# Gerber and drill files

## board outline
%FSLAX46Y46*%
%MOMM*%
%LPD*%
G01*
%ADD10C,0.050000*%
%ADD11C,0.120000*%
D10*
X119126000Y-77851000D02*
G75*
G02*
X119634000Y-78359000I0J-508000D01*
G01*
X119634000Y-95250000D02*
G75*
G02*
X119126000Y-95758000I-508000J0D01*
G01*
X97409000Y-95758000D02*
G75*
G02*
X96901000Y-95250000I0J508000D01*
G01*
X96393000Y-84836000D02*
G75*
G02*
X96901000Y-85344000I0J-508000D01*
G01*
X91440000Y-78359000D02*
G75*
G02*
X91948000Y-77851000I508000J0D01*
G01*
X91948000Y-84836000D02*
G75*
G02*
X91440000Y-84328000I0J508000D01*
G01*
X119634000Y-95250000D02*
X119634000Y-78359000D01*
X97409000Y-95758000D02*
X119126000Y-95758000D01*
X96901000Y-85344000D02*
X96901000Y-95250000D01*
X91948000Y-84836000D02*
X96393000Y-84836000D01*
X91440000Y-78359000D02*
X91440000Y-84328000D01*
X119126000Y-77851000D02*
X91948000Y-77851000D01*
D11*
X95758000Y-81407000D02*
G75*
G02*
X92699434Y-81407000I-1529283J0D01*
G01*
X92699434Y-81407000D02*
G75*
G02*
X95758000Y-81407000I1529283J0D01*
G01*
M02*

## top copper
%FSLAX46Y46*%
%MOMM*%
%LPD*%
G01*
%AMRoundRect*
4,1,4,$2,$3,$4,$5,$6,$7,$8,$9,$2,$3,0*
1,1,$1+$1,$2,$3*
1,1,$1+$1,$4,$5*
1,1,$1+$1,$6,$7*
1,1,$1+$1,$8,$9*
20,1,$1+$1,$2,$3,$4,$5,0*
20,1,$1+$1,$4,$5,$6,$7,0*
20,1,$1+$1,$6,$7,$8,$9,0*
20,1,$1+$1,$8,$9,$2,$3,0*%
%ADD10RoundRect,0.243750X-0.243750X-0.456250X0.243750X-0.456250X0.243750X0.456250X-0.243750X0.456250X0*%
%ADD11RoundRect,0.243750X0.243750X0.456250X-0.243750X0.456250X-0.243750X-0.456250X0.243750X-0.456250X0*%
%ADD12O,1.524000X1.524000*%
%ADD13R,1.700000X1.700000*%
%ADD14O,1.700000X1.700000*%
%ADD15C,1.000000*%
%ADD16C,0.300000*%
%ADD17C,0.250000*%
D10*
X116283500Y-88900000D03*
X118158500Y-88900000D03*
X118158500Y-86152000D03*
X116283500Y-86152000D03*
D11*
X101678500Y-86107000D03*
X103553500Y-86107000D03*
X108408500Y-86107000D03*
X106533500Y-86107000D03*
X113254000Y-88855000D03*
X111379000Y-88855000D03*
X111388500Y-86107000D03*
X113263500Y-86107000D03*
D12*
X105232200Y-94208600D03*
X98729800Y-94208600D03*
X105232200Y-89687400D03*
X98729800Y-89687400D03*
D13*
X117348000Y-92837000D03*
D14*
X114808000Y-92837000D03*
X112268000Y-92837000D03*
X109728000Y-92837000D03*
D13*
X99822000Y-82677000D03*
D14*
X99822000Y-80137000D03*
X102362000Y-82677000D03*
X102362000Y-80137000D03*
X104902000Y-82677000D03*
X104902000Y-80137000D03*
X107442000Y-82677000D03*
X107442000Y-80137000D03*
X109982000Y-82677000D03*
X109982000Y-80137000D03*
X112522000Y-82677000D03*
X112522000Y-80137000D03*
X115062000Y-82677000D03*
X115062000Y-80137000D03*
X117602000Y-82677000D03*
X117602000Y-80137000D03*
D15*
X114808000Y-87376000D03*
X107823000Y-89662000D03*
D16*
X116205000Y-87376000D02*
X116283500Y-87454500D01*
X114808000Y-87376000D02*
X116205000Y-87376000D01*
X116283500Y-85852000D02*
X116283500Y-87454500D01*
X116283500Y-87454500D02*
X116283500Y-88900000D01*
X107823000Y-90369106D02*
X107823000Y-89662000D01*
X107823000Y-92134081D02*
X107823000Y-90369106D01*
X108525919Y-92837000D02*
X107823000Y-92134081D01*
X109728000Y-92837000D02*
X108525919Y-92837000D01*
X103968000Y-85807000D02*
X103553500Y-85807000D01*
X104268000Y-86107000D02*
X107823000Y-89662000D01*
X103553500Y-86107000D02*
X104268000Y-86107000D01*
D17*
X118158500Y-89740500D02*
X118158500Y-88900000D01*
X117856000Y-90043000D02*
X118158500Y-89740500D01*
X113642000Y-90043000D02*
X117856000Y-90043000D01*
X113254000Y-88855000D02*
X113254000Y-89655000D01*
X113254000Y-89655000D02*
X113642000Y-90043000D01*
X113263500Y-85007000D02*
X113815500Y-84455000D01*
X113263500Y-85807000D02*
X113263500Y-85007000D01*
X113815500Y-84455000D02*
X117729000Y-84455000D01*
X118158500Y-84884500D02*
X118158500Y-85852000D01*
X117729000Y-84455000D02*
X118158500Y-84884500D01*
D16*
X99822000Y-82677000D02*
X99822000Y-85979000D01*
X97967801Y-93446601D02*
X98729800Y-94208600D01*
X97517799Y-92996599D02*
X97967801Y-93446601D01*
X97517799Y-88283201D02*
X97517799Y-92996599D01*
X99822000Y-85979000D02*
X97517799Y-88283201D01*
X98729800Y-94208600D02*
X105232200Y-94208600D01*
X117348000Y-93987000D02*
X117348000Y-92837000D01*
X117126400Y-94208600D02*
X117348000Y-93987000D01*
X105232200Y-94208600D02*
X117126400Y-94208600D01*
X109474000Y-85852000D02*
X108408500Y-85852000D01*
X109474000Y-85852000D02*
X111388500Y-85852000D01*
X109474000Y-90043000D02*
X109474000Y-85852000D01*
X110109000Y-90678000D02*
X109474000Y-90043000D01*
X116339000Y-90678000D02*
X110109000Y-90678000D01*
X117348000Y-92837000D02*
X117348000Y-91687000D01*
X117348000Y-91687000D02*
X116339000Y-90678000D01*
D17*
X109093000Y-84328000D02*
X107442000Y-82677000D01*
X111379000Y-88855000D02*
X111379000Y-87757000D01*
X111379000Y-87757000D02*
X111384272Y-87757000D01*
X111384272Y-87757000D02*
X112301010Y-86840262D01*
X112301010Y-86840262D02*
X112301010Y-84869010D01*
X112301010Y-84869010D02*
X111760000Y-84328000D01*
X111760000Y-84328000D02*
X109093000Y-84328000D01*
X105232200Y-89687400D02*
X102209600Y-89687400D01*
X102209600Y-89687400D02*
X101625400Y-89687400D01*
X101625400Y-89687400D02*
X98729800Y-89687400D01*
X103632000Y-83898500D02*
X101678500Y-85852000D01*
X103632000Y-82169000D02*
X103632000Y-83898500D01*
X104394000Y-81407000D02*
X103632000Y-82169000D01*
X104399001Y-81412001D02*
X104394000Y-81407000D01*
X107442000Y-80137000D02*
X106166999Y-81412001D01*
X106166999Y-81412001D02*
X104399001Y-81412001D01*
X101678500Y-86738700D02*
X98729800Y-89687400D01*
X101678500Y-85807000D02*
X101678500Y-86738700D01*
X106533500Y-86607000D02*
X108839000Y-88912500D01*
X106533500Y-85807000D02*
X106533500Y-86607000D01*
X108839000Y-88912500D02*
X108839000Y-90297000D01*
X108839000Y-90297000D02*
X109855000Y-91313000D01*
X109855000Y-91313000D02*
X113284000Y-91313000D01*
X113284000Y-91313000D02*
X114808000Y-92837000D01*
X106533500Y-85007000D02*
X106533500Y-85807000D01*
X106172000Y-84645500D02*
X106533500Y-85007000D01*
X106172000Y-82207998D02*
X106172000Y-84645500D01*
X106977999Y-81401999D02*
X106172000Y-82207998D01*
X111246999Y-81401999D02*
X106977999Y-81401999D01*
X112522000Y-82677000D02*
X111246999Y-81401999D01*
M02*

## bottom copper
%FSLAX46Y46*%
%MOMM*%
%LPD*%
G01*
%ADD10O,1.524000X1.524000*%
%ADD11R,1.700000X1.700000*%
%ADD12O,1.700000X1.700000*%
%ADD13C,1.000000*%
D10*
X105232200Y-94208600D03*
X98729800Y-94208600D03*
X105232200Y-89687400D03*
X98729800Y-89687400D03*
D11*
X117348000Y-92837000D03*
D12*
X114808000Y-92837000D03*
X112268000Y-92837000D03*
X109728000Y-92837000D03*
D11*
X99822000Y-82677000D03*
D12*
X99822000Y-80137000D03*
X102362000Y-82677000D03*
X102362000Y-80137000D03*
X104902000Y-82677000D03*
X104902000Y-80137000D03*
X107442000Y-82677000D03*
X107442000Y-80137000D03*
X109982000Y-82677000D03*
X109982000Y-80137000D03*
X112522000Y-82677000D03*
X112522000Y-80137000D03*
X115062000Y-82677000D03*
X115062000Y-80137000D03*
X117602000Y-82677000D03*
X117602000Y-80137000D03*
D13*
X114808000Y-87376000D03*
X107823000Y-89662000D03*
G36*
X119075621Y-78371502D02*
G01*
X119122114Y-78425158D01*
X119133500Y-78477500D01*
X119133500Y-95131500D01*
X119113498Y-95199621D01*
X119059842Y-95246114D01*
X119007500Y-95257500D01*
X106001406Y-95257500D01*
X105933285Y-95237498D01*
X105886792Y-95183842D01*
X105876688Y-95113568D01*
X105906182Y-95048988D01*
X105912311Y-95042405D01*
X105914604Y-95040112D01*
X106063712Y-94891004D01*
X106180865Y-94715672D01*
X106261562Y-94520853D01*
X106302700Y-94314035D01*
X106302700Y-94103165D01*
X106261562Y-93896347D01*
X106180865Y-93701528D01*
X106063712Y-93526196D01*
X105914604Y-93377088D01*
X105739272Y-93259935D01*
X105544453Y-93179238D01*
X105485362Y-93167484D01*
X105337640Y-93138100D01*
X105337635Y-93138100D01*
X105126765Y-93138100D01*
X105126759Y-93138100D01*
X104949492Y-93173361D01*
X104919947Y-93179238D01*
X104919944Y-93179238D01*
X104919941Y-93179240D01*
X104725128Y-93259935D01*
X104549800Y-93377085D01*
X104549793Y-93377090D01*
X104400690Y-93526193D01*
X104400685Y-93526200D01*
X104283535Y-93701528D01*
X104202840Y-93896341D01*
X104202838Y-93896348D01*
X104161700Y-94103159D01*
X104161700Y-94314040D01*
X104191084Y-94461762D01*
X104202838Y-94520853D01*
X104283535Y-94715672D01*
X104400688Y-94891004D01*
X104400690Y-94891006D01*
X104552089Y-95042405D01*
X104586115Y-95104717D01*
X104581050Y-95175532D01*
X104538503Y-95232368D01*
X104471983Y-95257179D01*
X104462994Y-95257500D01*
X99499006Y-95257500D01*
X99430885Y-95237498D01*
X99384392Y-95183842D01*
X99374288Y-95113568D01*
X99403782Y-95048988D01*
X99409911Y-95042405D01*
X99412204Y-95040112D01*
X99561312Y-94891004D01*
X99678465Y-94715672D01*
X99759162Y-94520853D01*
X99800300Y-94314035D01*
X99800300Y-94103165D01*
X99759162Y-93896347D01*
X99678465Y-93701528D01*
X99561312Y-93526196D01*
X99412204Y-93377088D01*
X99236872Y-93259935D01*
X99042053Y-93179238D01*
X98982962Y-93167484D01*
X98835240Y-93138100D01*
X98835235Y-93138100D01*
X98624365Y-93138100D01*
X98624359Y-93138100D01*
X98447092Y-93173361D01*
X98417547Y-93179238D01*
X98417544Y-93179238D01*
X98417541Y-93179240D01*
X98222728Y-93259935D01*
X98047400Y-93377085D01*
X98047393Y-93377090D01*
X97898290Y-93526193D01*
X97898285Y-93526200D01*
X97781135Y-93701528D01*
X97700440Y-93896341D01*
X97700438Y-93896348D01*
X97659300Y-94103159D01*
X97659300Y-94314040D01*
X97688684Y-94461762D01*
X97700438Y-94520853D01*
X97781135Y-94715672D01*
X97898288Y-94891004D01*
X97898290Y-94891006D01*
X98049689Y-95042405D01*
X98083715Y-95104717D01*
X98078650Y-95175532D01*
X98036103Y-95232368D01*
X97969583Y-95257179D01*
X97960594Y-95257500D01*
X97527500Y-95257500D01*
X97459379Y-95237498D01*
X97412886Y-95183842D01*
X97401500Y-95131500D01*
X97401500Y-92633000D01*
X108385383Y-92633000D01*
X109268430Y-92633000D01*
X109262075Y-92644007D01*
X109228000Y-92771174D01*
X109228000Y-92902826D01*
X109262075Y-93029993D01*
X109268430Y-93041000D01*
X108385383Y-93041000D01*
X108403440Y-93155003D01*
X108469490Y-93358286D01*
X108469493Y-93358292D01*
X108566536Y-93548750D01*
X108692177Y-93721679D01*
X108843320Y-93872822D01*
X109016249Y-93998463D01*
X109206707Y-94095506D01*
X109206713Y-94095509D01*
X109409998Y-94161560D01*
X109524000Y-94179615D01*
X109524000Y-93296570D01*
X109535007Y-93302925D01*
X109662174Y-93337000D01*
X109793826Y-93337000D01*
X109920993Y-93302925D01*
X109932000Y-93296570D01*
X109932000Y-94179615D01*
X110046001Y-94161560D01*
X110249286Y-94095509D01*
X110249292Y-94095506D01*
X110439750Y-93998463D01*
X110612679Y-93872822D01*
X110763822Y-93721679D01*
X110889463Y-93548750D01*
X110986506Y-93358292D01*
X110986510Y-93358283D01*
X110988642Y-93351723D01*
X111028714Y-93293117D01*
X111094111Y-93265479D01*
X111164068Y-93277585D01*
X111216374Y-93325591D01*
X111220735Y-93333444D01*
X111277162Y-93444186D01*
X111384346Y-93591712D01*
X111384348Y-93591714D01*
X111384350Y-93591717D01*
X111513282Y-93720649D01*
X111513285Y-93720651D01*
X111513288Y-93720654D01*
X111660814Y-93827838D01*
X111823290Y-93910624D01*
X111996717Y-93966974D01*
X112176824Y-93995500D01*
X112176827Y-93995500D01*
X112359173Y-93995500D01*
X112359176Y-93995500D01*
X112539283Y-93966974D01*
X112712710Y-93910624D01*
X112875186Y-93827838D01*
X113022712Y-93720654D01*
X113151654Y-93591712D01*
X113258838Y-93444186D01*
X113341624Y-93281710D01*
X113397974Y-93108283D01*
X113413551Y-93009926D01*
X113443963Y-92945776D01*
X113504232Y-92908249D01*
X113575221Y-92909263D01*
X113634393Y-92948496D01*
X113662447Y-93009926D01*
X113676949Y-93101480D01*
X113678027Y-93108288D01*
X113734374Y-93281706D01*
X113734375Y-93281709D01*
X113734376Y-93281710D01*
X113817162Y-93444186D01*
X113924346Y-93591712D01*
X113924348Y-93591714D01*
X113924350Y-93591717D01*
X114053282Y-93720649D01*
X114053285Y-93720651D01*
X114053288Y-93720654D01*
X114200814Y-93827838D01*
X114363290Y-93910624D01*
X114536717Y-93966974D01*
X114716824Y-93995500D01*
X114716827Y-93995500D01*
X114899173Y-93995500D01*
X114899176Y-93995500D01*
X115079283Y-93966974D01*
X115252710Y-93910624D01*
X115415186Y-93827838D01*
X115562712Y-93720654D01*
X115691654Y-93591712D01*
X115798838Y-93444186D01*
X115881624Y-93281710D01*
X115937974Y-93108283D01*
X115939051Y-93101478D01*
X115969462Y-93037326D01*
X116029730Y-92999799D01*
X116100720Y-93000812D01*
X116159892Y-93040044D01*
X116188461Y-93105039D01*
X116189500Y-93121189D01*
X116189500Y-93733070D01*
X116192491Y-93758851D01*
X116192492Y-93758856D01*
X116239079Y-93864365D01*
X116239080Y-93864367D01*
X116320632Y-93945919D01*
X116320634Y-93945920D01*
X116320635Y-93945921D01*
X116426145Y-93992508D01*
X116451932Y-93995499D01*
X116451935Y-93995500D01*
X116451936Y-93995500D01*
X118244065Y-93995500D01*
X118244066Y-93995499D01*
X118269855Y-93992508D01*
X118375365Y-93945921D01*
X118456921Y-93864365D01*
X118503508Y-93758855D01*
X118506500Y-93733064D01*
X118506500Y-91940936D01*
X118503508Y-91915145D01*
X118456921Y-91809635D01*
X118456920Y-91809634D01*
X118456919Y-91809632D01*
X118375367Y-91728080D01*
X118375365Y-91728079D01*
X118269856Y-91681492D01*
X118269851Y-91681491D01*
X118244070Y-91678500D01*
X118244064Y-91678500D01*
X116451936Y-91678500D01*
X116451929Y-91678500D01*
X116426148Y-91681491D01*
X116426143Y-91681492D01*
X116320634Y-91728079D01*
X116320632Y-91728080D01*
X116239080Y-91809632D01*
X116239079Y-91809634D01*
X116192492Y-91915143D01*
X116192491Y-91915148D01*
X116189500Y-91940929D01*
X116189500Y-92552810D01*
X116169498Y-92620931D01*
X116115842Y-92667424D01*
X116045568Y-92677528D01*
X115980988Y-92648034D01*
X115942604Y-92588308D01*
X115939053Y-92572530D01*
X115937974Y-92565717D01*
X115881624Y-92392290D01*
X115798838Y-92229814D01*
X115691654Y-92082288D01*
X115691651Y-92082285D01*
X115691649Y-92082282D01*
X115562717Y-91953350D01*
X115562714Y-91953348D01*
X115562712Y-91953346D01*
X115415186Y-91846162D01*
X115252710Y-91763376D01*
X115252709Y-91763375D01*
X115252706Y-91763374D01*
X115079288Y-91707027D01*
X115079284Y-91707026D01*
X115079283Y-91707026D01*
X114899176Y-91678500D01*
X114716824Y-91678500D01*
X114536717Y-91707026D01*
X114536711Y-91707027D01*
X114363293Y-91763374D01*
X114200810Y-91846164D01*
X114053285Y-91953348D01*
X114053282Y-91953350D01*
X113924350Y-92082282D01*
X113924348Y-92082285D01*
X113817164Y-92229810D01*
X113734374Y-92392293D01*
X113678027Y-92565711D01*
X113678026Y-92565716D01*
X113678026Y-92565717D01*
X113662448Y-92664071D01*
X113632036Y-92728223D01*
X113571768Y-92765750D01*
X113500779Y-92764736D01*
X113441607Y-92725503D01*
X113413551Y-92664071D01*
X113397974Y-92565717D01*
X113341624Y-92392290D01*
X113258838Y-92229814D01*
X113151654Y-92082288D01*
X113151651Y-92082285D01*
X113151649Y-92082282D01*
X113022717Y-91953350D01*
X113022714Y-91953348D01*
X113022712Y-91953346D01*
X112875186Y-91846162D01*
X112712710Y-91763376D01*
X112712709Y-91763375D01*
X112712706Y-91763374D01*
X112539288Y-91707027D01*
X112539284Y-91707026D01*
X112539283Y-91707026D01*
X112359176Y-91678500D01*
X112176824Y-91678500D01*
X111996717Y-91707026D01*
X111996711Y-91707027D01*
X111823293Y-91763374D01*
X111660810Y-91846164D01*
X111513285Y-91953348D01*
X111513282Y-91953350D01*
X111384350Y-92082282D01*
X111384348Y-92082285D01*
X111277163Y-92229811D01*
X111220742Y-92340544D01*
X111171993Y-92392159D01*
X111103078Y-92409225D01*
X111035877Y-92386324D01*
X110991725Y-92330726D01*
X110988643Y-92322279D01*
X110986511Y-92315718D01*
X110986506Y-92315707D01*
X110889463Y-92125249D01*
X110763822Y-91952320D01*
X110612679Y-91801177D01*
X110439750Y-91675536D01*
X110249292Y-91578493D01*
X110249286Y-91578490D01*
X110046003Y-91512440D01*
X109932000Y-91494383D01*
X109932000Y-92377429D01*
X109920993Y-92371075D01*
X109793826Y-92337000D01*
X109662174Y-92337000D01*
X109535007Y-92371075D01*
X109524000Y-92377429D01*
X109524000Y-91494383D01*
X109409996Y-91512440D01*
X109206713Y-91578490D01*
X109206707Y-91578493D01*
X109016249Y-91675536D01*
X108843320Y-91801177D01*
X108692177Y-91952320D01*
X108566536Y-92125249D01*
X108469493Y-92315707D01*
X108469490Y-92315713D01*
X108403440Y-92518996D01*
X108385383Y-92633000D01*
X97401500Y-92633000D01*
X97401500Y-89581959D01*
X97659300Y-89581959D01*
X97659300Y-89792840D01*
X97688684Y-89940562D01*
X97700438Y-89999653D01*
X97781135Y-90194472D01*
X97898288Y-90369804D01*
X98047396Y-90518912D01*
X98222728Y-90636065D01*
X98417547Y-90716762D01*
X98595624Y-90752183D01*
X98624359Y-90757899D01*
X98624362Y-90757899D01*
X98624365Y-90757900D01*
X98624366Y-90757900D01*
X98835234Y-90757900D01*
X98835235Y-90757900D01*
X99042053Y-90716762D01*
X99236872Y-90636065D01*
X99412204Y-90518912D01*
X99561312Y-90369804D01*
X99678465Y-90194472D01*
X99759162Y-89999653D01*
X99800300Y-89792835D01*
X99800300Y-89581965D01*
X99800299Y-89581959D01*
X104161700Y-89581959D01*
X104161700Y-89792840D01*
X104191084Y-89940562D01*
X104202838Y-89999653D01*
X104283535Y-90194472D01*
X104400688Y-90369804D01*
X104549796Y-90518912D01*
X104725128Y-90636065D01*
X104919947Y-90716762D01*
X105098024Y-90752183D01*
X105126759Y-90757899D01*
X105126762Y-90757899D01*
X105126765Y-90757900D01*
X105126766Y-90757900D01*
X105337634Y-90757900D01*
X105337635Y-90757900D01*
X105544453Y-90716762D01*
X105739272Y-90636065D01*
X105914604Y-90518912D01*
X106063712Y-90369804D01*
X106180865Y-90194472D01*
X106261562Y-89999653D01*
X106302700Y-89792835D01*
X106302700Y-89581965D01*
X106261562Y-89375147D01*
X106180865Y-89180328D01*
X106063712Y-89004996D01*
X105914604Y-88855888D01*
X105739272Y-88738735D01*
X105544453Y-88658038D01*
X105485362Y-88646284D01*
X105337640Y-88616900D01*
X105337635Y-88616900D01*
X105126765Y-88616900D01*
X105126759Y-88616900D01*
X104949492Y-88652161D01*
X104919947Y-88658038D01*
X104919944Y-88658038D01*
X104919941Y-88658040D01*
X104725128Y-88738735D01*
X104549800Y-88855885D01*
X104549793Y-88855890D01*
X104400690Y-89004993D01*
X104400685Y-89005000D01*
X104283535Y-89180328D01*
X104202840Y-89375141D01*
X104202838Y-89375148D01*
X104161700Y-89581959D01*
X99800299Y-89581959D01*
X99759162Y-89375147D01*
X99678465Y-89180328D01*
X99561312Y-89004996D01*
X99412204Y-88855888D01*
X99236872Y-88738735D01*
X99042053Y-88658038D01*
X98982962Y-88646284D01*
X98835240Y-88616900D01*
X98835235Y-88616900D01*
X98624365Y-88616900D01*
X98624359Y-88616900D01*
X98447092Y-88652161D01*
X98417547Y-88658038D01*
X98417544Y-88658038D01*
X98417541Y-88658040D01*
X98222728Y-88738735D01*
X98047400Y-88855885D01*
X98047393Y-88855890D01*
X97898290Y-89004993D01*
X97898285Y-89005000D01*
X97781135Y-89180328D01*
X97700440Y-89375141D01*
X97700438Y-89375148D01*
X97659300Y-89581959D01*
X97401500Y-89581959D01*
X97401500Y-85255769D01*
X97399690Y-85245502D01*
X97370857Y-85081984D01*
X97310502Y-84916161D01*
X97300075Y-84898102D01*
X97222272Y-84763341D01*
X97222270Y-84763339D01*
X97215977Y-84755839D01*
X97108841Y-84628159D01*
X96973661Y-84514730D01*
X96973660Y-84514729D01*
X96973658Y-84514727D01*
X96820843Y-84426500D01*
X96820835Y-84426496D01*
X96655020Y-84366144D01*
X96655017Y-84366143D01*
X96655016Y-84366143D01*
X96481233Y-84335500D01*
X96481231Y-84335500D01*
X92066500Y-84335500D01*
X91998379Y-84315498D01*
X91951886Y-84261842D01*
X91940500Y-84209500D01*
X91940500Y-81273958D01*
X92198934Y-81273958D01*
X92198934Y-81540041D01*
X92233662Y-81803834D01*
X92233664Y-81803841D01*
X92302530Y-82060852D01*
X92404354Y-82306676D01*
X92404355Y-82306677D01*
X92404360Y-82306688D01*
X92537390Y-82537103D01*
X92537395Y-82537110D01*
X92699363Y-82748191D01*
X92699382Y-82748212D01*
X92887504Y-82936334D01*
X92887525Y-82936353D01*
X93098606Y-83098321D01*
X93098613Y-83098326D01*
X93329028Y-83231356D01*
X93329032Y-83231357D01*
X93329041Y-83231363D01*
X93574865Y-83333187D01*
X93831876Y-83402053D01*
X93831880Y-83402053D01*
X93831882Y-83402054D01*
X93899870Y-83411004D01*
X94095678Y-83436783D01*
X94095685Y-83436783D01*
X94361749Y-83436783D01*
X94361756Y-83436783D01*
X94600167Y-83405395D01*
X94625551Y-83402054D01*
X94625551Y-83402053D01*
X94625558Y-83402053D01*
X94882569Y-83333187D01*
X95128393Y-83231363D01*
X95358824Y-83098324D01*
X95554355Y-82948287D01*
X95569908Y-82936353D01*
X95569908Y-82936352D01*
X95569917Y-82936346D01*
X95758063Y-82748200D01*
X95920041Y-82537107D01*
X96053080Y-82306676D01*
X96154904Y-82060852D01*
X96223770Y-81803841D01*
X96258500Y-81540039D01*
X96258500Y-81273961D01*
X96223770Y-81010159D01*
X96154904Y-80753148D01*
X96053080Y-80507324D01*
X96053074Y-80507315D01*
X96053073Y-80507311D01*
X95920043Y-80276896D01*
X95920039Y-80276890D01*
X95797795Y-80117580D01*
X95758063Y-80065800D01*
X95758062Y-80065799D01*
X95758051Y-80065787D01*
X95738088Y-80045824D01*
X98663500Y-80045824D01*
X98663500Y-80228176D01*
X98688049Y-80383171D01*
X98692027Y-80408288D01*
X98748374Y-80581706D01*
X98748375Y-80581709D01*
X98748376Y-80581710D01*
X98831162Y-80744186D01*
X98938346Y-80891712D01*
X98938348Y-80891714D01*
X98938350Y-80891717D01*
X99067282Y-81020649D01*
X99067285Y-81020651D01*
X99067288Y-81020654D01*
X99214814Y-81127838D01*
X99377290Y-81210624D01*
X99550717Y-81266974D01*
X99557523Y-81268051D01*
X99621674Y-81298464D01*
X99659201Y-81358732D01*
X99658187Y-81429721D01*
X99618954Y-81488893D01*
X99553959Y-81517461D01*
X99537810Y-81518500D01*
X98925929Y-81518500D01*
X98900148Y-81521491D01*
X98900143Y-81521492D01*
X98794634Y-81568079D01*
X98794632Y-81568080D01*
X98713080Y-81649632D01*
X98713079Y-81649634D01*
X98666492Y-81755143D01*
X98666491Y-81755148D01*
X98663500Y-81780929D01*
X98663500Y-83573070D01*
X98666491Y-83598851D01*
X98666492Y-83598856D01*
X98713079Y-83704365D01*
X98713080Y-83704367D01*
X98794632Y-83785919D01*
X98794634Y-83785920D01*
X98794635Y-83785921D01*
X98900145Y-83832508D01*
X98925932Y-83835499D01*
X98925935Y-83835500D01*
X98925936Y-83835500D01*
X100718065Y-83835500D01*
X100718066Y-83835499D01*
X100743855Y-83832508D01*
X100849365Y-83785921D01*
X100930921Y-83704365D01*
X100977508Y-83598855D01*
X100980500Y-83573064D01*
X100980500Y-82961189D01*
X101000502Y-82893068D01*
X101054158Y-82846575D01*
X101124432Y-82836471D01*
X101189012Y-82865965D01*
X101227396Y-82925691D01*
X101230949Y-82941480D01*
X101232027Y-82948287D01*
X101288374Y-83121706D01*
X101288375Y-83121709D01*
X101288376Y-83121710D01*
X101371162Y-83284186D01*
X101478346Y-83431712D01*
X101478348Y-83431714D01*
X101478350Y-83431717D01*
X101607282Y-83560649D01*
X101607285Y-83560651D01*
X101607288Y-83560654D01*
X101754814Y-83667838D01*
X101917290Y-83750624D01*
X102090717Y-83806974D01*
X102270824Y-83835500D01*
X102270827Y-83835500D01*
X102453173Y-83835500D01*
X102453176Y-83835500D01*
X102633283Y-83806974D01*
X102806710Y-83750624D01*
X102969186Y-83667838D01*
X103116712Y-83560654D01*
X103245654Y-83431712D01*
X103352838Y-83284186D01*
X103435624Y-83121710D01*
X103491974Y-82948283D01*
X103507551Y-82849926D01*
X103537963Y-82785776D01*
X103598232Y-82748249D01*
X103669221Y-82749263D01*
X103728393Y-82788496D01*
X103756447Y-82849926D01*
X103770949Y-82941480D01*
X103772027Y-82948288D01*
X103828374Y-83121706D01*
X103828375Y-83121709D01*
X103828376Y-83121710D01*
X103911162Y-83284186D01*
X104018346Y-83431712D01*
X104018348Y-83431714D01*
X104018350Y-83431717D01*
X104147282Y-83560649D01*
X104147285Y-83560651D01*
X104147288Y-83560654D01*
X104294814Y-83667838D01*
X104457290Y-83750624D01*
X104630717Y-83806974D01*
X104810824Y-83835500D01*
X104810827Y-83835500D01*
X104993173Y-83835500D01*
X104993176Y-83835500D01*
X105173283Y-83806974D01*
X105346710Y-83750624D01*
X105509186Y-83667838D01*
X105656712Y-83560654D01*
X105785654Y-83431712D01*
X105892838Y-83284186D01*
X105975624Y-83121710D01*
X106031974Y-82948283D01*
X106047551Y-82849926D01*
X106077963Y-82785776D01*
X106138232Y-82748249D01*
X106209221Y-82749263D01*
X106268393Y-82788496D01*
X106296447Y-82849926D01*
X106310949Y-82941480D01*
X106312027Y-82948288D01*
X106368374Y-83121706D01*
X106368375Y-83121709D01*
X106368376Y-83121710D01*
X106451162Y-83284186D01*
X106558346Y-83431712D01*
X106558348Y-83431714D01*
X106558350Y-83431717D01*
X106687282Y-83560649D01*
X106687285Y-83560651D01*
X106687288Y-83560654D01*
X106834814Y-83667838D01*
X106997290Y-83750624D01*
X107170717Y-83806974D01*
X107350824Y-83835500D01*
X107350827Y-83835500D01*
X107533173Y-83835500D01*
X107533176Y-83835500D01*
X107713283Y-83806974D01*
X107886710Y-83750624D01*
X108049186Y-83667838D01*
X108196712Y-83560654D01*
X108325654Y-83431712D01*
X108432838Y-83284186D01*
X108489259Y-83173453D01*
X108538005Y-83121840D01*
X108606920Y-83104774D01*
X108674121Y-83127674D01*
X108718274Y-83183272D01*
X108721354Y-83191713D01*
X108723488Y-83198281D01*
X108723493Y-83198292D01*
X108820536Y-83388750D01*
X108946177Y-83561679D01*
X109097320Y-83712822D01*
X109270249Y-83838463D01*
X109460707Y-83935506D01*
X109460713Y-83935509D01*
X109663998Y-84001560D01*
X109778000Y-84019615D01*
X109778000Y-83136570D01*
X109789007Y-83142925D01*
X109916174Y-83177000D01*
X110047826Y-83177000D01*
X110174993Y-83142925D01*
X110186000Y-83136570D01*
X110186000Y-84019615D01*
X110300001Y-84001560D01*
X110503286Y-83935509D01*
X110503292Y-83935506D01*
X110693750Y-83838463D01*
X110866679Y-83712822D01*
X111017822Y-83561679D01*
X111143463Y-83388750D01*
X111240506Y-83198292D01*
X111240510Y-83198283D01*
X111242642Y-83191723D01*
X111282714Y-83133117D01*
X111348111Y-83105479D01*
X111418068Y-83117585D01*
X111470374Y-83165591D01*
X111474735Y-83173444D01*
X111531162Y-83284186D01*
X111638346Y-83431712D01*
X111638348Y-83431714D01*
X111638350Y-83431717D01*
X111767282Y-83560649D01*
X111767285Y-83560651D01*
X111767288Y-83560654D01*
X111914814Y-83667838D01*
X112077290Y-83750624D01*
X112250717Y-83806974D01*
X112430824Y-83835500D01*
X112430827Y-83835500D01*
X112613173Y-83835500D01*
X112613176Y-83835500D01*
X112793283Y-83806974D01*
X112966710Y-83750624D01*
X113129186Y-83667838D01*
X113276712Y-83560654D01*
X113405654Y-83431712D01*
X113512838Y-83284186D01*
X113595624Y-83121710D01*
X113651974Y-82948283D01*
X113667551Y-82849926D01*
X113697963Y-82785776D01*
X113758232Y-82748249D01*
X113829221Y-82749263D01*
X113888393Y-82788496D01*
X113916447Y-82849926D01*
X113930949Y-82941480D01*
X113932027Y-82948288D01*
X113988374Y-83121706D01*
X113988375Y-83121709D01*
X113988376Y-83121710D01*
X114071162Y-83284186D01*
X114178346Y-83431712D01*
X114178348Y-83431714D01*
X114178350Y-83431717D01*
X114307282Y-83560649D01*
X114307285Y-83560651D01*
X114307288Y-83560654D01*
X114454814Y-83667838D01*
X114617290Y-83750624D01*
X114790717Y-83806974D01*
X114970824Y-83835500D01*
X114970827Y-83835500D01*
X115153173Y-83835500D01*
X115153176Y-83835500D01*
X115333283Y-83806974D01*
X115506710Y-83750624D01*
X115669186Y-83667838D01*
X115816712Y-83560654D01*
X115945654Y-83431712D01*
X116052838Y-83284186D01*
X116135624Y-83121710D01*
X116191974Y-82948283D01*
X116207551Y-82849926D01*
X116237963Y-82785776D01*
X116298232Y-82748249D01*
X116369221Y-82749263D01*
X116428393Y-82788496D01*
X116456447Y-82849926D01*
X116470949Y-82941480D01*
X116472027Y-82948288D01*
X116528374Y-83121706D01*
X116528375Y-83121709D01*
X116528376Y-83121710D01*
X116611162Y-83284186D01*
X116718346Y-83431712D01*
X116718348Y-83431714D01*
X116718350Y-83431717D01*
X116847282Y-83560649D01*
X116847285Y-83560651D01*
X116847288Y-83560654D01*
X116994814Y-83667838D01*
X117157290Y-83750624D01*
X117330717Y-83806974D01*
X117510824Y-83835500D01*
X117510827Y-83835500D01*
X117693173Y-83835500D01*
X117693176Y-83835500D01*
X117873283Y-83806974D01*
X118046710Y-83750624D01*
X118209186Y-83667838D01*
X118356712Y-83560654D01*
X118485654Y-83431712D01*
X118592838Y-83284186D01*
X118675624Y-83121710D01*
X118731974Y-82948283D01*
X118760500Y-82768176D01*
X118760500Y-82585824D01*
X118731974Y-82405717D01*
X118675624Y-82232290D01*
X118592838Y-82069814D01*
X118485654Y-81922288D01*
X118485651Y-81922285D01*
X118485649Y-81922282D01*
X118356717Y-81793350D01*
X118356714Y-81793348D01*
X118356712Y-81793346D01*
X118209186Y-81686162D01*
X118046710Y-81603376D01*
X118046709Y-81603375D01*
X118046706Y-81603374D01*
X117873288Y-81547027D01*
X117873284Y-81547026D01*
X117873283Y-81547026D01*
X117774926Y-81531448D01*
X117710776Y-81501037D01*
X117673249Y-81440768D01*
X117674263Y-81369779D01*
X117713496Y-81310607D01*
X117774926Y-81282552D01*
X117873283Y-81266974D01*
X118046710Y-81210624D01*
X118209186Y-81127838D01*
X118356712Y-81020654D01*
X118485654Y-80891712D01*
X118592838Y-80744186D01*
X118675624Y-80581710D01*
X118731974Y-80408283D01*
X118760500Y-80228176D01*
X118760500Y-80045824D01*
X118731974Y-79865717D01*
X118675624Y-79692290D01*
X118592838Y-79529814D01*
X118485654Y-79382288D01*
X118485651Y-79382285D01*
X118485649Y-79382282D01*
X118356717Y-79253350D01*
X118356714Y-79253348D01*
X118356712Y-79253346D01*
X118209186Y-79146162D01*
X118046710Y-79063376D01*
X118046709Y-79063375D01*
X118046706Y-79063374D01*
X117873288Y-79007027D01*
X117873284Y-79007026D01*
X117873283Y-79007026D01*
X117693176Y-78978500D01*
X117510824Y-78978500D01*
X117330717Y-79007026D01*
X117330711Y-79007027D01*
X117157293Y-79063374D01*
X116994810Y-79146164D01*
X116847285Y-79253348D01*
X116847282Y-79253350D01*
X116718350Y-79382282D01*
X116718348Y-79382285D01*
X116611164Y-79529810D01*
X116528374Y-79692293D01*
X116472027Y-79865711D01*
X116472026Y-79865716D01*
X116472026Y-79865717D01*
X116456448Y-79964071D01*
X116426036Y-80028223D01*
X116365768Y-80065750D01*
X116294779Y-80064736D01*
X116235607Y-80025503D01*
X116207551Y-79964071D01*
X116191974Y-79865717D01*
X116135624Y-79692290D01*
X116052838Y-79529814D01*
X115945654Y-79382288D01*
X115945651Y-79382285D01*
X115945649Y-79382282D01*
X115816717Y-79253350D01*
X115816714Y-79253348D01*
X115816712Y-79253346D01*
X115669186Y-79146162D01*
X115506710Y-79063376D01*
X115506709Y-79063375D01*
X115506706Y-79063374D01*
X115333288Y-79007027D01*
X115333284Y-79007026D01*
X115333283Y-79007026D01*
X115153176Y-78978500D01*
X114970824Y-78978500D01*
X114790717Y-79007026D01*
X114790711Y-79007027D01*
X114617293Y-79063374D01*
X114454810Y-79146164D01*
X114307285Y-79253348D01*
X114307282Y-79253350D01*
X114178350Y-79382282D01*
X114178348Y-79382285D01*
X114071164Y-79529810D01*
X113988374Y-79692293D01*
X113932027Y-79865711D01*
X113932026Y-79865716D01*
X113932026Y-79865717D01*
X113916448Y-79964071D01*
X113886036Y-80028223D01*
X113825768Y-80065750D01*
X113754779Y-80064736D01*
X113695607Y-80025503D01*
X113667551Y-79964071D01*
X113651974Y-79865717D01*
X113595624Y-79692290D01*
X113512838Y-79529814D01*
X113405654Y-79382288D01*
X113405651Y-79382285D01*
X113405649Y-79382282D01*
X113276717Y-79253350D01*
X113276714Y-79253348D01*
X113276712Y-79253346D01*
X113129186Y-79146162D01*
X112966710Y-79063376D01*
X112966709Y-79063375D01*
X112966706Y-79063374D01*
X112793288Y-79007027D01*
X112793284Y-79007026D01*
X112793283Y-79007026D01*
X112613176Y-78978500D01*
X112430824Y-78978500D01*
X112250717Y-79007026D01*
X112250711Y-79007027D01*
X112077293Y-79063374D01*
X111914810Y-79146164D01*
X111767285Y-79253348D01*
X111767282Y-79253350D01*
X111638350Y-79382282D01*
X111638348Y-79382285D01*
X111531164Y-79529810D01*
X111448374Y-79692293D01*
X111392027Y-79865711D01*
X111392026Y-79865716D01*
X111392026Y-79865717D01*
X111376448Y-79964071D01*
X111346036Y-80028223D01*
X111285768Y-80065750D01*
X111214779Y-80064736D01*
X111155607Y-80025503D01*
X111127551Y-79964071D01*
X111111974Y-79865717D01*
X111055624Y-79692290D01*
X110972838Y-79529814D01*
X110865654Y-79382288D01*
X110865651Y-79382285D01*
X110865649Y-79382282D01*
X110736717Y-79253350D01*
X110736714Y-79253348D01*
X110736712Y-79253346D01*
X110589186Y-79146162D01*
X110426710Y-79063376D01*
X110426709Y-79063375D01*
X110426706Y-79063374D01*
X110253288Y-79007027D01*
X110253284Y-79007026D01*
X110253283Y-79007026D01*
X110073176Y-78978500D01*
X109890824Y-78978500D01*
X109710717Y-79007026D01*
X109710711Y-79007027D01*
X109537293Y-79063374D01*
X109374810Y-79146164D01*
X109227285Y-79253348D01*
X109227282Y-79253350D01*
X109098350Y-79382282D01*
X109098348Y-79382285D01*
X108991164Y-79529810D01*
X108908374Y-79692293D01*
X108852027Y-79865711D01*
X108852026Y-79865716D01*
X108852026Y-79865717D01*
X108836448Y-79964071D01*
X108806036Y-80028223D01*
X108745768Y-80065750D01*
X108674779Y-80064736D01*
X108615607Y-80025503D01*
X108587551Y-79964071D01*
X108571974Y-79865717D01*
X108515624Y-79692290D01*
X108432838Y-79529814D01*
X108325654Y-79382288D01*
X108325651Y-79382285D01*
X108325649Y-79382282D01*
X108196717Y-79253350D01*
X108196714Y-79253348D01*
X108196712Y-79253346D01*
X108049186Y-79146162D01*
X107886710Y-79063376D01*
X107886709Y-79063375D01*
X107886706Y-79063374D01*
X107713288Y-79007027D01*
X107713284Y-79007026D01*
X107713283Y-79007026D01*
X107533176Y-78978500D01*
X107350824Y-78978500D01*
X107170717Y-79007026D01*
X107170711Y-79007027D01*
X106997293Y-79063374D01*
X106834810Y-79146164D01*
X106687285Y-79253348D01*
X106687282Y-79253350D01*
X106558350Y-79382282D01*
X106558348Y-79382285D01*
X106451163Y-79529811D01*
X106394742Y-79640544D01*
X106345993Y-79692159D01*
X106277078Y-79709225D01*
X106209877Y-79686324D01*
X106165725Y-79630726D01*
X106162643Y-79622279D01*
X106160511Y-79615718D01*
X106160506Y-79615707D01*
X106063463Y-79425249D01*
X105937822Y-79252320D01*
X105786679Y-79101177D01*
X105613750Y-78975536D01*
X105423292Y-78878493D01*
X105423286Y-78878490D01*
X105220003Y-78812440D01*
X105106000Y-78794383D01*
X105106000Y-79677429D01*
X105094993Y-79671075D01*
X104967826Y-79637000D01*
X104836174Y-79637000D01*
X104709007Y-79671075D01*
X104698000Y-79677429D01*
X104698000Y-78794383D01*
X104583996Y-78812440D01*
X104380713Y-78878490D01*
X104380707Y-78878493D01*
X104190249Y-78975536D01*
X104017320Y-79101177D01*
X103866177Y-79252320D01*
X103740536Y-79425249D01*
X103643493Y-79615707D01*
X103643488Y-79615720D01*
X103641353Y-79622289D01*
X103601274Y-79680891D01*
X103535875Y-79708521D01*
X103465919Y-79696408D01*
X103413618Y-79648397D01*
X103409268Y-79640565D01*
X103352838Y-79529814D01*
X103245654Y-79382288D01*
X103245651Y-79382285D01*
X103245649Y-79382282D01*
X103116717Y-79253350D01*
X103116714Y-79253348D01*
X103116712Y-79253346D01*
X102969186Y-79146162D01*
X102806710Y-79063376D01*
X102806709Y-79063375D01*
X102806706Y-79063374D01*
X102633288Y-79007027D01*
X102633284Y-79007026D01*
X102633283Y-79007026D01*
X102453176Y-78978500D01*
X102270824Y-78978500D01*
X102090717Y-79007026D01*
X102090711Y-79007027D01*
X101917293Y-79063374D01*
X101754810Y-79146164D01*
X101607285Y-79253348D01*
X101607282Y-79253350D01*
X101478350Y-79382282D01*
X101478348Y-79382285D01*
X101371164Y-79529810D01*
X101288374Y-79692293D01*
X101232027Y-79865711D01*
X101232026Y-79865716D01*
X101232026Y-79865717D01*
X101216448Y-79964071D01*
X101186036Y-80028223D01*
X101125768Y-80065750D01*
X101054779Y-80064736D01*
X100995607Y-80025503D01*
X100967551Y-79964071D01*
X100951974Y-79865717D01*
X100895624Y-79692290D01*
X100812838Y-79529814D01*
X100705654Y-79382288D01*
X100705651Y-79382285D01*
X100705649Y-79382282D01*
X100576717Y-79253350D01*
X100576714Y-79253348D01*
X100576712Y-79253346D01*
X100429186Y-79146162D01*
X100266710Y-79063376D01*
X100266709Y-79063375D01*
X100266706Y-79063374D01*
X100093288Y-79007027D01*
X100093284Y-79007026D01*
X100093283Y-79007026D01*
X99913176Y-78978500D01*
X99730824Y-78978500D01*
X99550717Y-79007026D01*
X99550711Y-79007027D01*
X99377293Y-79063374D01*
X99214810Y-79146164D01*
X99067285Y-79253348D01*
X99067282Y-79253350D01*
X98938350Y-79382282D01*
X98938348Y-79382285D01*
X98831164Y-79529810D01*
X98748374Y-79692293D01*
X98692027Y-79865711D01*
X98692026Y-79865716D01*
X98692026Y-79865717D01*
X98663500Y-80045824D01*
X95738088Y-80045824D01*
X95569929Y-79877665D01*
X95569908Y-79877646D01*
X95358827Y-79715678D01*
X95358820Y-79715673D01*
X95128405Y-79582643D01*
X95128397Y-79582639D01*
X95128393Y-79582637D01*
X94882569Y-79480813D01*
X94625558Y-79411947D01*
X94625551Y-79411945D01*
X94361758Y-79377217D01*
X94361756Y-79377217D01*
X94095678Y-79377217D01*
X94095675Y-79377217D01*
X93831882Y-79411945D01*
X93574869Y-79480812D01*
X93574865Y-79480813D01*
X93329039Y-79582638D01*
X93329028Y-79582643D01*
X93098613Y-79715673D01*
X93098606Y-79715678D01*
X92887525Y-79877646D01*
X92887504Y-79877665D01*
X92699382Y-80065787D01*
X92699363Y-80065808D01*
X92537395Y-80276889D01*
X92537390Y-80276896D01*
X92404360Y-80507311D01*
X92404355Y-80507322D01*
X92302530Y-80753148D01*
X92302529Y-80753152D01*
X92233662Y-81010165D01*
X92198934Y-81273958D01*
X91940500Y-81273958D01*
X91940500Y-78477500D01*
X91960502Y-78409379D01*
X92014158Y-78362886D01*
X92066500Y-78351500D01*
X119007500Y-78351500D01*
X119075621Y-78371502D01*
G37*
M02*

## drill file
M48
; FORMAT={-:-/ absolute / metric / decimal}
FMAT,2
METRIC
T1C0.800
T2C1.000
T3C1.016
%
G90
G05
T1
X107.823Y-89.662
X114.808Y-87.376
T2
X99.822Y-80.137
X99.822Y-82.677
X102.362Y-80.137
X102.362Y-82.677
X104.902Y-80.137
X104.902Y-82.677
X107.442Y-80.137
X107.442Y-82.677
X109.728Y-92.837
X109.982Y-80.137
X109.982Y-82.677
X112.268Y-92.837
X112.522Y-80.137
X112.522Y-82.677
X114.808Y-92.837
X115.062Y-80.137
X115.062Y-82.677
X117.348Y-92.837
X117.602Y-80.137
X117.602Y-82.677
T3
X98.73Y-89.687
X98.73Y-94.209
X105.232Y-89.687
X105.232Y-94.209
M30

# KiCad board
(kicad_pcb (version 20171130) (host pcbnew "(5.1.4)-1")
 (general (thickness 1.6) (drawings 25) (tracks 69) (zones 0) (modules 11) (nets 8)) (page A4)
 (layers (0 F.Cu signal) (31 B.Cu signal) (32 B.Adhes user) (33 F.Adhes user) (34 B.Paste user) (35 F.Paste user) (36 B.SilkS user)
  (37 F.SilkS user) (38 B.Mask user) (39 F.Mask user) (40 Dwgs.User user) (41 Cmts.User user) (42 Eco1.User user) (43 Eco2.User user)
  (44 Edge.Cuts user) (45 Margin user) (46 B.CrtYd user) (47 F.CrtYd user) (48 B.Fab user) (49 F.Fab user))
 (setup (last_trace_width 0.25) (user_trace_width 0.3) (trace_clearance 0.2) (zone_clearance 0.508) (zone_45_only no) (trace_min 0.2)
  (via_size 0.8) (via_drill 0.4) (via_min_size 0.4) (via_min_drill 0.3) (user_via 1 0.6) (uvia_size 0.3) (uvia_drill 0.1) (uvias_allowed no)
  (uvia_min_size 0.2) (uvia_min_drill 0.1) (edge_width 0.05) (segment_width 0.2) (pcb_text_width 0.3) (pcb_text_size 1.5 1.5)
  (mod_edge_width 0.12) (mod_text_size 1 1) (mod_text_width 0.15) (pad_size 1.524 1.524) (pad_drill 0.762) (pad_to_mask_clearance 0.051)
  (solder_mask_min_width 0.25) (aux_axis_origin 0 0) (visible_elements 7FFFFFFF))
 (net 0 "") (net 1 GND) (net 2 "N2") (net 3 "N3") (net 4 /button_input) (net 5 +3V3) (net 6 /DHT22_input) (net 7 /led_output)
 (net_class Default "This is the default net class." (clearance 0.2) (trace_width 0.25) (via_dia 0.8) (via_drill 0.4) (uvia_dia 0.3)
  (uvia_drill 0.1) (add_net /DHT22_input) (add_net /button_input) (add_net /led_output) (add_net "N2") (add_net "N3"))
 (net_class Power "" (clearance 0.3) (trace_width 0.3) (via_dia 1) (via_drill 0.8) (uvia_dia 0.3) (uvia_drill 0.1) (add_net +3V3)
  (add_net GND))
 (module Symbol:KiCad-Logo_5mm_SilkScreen (layer B.Cu) (at 105.918 89.916 180)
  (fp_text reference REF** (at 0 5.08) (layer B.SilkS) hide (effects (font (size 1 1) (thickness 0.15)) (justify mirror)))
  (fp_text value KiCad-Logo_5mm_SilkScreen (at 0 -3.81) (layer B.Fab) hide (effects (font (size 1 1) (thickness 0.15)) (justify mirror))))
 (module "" (layer F.Cu) (at 116.332 98.171)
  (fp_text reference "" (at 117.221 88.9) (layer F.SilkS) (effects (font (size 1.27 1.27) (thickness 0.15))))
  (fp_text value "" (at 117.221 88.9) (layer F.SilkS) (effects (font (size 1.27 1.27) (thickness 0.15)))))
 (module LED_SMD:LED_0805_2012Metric (layer F.Cu) (at 117.221 88.9)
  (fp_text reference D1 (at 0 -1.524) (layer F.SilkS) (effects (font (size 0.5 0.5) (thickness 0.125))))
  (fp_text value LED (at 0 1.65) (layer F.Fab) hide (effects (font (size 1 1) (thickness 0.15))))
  (pad 1 smd roundrect (at -0.9375 0) (size 0.975 1.4) (layers F.Cu F.Paste F.Mask) (roundrect_rratio 0.25) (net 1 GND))
  (pad 2 smd roundrect (at 0.9375 0) (size 0.975 1.4) (layers F.Cu F.Paste F.Mask) (roundrect_rratio 0.25) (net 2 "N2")))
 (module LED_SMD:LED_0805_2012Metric (layer F.Cu) (at 117.221 86.152)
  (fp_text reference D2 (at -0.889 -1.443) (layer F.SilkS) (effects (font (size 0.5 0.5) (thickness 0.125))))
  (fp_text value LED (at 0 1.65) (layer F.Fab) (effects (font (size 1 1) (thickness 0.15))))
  (pad 2 smd roundrect (at 0.9375 0) (size 0.975 1.4) (layers F.Cu F.Paste F.Mask) (roundrect_rratio 0.25) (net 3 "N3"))
  (pad 1 smd roundrect (at -0.9375 0) (size 0.975 1.4) (layers F.Cu F.Paste F.Mask) (roundrect_rratio 0.25) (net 1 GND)))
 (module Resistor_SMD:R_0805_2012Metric (layer F.Cu) (at 102.616 86.107 180)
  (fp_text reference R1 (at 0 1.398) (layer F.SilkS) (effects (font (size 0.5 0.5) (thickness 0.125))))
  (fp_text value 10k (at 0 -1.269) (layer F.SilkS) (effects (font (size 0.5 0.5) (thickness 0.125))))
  (pad 2 smd roundrect (at 0.9375 0 180) (size 0.975 1.4) (layers F.Cu F.Paste F.Mask) (roundrect_rratio 0.25) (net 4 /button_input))
  (pad 1 smd roundrect (at -0.9375 0 180) (size 0.975 1.4) (layers F.Cu F.Paste F.Mask) (roundrect_rratio 0.25) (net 1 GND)))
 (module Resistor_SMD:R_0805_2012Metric (layer F.Cu) (at 107.471 86.107 180)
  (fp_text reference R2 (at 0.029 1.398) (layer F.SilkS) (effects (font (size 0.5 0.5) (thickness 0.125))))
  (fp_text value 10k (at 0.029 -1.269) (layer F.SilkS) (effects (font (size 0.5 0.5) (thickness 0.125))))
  (pad 1 smd roundrect (at -0.9375 0 180) (size 0.975 1.4) (layers F.Cu F.Paste F.Mask) (roundrect_rratio 0.25) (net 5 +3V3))
  (pad 2 smd roundrect (at 0.9375 0 180) (size 0.975 1.4) (layers F.Cu F.Paste F.Mask) (roundrect_rratio 0.25) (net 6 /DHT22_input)))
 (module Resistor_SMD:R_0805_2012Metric (layer F.Cu) (at 112.3165 88.855 180)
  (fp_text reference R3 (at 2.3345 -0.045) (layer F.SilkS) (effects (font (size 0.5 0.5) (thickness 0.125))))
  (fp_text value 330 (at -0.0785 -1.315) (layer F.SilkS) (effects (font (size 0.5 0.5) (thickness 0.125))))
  (pad 1 smd roundrect (at -0.9375 0 180) (size 0.975 1.4) (layers F.Cu F.Paste F.Mask) (roundrect_rratio 0.25) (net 2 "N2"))
  (pad 2 smd roundrect (at 0.9375 0 180) (size 0.975 1.4) (layers F.Cu F.Paste F.Mask) (roundrect_rratio 0.25) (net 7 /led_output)))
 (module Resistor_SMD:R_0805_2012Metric (layer F.Cu) (at 112.326 86.107 180)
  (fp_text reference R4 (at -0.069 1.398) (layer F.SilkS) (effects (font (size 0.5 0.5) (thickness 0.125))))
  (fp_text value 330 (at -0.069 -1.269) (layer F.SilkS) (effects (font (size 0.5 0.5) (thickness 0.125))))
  (pad 2 smd roundrect (at 0.9375 0 180) (size 0.975 1.4) (layers F.Cu F.Paste F.Mask) (roundrect_rratio 0.25) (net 5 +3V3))
  (pad 1 smd roundrect (at -0.9375 0 180) (size 0.975 1.4) (layers F.Cu F.Paste F.Mask) (roundrect_rratio 0.25) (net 3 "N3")))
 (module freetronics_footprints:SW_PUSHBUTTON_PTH (layer F.Cu) (at 101.981 91.948 180)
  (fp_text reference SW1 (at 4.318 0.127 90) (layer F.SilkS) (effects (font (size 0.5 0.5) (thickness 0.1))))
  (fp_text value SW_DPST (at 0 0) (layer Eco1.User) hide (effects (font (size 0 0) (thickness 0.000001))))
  (pad 1 thru_hole oval (at -3.2512 -2.2606 180) (size 1.524 1.524) (drill 1.016) (layers *.Cu *.Mask) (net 5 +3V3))
  (pad 1 thru_hole oval (at 3.2512 -2.2606 180) (size 1.524 1.524) (drill 1.016) (layers *.Cu *.Mask) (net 5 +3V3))
  (pad 2 thru_hole oval (at -3.2512 2.2606 180) (size 1.524 1.524) (drill 1.016) (layers *.Cu *.Mask) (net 4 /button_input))
  (pad 2 thru_hole oval (at 3.2512 2.2606 180) (size 1.524 1.524) (drill 1.016) (layers *.Cu *.Mask) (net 4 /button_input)))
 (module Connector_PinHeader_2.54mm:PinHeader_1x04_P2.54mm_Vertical (layer F.Cu) (at 117.348 92.837 270)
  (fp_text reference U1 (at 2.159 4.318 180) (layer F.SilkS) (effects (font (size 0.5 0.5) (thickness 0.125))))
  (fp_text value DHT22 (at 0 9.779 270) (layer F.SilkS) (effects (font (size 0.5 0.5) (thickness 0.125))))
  (pad 1 thru_hole rect (at 0 0 270) (size 1.7 1.7) (drill 1) (layers *.Cu *.Mask) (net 5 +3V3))
  (pad 2 thru_hole oval (at 0 2.54 270) (size 1.7 1.7) (drill 1) (layers *.Cu *.Mask) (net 6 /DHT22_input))
  (pad 3 thru_hole oval (at 0 5.08 270) (size 1.7 1.7) (drill 1) (layers *.Cu *.Mask))
  (pad 4 thru_hole oval (at 0 7.62 270) (size 1.7 1.7) (drill 1) (layers *.Cu *.Mask) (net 1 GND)))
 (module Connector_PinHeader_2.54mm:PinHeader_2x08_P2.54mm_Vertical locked (layer F.Cu) (at 99.822 82.677 90)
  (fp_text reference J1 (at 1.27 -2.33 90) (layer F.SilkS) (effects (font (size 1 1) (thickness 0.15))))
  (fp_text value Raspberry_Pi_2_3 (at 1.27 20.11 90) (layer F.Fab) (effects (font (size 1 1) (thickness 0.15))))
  (pad 1 thru_hole rect (at 0 0 90) (size 1.7 1.7) (drill 1) (layers *.Cu *.Mask) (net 5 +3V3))
  (pad 2 thru_hole oval (at 2.54 0 90) (size 1.7 1.7) (drill 1) (layers *.Cu *.Mask))
  (pad 3 thru_hole oval (at 0 2.54 90) (size 1.7 1.7) (drill 1) (layers *.Cu *.Mask))
  (pad 4 thru_hole oval (at 2.54 2.54 90) (size 1.7 1.7) (drill 1) (layers *.Cu *.Mask))
  (pad 5 thru_hole oval (at 0 5.08 90) (size 1.7 1.7) (drill 1) (layers *.Cu *.Mask))
  (pad 6 thru_hole oval (at 2.54 5.08 90) (size 1.7 1.7) (drill 1) (layers *.Cu *.Mask) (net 1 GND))
  (pad 7 thru_hole oval (at 0 7.62 90) (size 1.7 1.7) (drill 1) (layers *.Cu *.Mask) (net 7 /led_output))
  (pad 8 thru_hole oval (at 2.54 7.62 90) (size 1.7 1.7) (drill 1) (layers *.Cu *.Mask) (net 4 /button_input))
  (pad 9 thru_hole oval (at 0 10.16 90) (size 1.7 1.7) (drill 1) (layers *.Cu *.Mask) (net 1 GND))
  (pad 10 thru_hole oval (at 2.54 10.16 90) (size 1.7 1.7) (drill 1) (layers *.Cu *.Mask))
  (pad 11 thru_hole oval (at 0 12.7 90) (size 1.7 1.7) (drill 1) (layers *.Cu *.Mask) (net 6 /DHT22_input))
  (pad 12 thru_hole oval (at 2.54 12.7 90) (size 1.7 1.7) (drill 1) (layers *.Cu *.Mask))
  (pad 13 thru_hole oval (at 0 15.24 90) (size 1.7 1.7) (drill 1) (layers *.Cu *.Mask))
  (pad 14 thru_hole oval (at 2.54 15.24 90) (size 1.7 1.7) (drill 1) (layers *.Cu *.Mask))
  (pad 15 thru_hole oval (at 0 17.78 90) (size 1.7 1.7) (drill 1) (layers *.Cu *.Mask))
  (pad 16 thru_hole oval (at 2.54 17.78 90) (size 1.7 1.7) (drill 1) (layers *.Cu *.Mask)))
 (gr_arc (start 119.126 78.359) (end 119.634 78.359) (angle -90) (layer Edge.Cuts) (width 0.05))
 (gr_arc (start 119.126 95.25) (end 119.126 95.758) (angle -90) (layer Edge.Cuts) (width 0.05))
 (gr_arc (start 97.409 95.25) (end 96.901 95.25) (angle -90) (layer Edge.Cuts) (width 0.05))
 (gr_arc (start 96.393 85.344) (end 96.901 85.344) (angle -90) (layer Edge.Cuts) (width 0.05))
 (gr_arc (start 91.948 78.359) (end 91.948 77.851) (angle -90) (layer Edge.Cuts) (width 0.05))
 (gr_arc (start 91.948 84.328) (end 91.44 84.328) (angle -90) (layer Edge.Cuts) (width 0.05))
 (gr_line (start 119.634 95.25) (end 119.634 78.359) (layer Edge.Cuts) (width 0.05))
 (gr_line (start 97.409 95.758) (end 119.126 95.758) (layer Edge.Cuts) (width 0.05))
 (gr_line (start 96.901 85.344) (end 96.901 95.25) (layer Edge.Cuts) (width 0.05))
 (gr_line (start 91.948 84.836) (end 96.393 84.836) (layer Edge.Cuts) (width 0.05))
 (gr_line (start 91.44 78.359) (end 91.44 84.328) (layer Edge.Cuts) (width 0.05))
 (gr_line (start 119.126 77.851) (end 91.948 77.851) (layer Edge.Cuts) (width 0.05))
 (gr_circle (center 94.228717 81.407) (end 95.758 81.407) (layer Edge.Cuts) (width 0.12))
 (via (at 114.808 87.376) (size 1) (drill 0.8) (layers F.Cu B.Cu) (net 1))
 (segment (start 116.205 87.376) (end 116.2835 87.4545) (width 0.3) (layer F.Cu) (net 1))
 (segment (start 114.808 87.376) (end 116.205 87.376) (width 0.3) (layer F.Cu) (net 1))
 (segment (start 116.2835 85.852) (end 116.2835 87.4545) (width 0.3) (layer F.Cu) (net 1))
 (segment (start 116.2835 87.4545) (end 116.2835 88.9) (width 0.3) (layer F.Cu) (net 1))
 (via (at 107.823 89.662) (size 1) (drill 0.8) (layers F.Cu B.Cu) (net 1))
 (segment (start 107.823 90.369106) (end 107.823 89.662) (width 0.3) (layer F.Cu) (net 1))
 (segment (start 107.823 92.134081) (end 107.823 90.369106) (width 0.3) (layer F.Cu) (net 1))
 (segment (start 108.525919 92.837) (end 107.823 92.134081) (width 0.3) (layer F.Cu) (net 1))
 (segment (start 109.728 92.837) (end 108.525919 92.837) (width 0.3) (layer F.Cu) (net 1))
 (segment (start 103.968 85.807) (end 103.5535 85.807) (width 0.3) (layer F.Cu) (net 1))
 (segment (start 104.268 86.107) (end 107.823 89.662) (width 0.3) (layer F.Cu) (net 1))
 (segment (start 103.5535 86.107) (end 104.268 86.107) (width 0.3) (layer F.Cu) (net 1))
 (segment (start 118.1585 89.7405) (end 118.1585 88.9) (width 0.25) (layer F.Cu) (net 2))
 (segment (start 117.856 90.043) (end 118.1585 89.7405) (width 0.25) (layer F.Cu) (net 2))
 (segment (start 113.642 90.043) (end 117.856 90.043) (width 0.25) (layer F.Cu) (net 2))
 (segment (start 113.254 88.855) (end 113.254 89.655) (width 0.25) (layer F.Cu) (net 2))
 (segment (start 113.254 89.655) (end 113.642 90.043) (width 0.25) (layer F.Cu) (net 2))
 (segment (start 113.2635 85.007) (end 113.8155 84.455) (width 0.25) (layer F.Cu) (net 3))
 (segment (start 113.2635 85.807) (end 113.2635 85.007) (width 0.25) (layer F.Cu) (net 3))
 (segment (start 113.8155 84.455) (end 117.729 84.455) (width 0.25) (layer F.Cu) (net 3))
 (segment (start 118.1585 84.8845) (end 118.1585 85.852) (width 0.25) (layer F.Cu) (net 3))
 (segment (start 117.729 84.455) (end 118.1585 84.8845) (width 0.25) (layer F.Cu) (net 3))
 (segment (start 99.822 82.677) (end 99.822 85.979) (width 0.3) (layer F.Cu) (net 5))
 (segment (start 97.967801 93.446601) (end 98.7298 94.2086) (width 0.3) (layer F.Cu) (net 5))
 (segment (start 97.517799 92.996599) (end 97.967801 93.446601) (width 0.3) (layer F.Cu) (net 5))
 (segment (start 97.517799 88.283201) (end 97.517799 92.996599) (width 0.3) (layer F.Cu) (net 5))
 (segment (start 99.822 85.979) (end 97.517799 88.283201) (width 0.3) (layer F.Cu) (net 5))
 (segment (start 98.7298 94.2086) (end 105.2322 94.2086) (width 0.3) (layer F.Cu) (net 5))
 (segment (start 117.348 93.987) (end 117.348 92.837) (width 0.3) (layer F.Cu) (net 5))
 (segment (start 117.1264 94.2086) (end 117.348 93.987) (width 0.3) (layer F.Cu) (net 5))
 (segment (start 105.2322 94.2086) (end 117.1264 94.2086) (width 0.3) (layer F.Cu) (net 5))
 (segment (start 109.474 85.852) (end 108.4085 85.852) (width 0.3) (layer F.Cu) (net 5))
 (segment (start 109.474 85.852) (end 111.3885 85.852) (width 0.3) (layer F.Cu) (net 5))
 (segment (start 109.474 90.043) (end 109.474 85.852) (width 0.3) (layer F.Cu) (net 5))
 (segment (start 110.109 90.678) (end 109.474 90.043) (width 0.3) (layer F.Cu) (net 5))
 (segment (start 116.339 90.678) (end 110.109 90.678) (width 0.3) (layer F.Cu) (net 5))
 (segment (start 117.348 92.837) (end 117.348 91.687) (width 0.3) (layer F.Cu) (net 5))
 (segment (start 117.348 91.687) (end 116.339 90.678) (width 0.3) (layer F.Cu) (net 5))
 (segment (start 109.093 84.328) (end 107.442 82.677) (width 0.25) (layer F.Cu) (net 7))
 (segment (start 111.379 88.855) (end 111.379 87.757) (width 0.25) (layer F.Cu) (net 7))
 (segment (start 111.379 87.757) (end 111.384272 87.757) (width 0.25) (layer F.Cu) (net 7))
 (segment (start 111.384272 87.757) (end 112.30101 86.840262) (width 0.25) (layer F.Cu) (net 7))
 (segment (start 112.30101 86.840262) (end 112.30101 84.86901) (width 0.25) (layer F.Cu) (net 7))
 (segment (start 112.30101 84.86901) (end 111.76 84.328) (width 0.25) (layer F.Cu) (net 7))
 (segment (start 111.76 84.328) (end 109.093 84.328) (width 0.25) (layer F.Cu) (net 7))
 (segment (start 105.2322 89.6874) (end 102.2096 89.6874) (width 0.25) (layer F.Cu) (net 4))
 (segment (start 102.2096 89.6874) (end 101.6254 89.6874) (width 0.25) (layer F.Cu) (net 4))
 (segment (start 101.6254 89.6874) (end 98.7298 89.6874) (width 0.25) (layer F.Cu) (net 4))
 (segment (start 103.632 83.8985) (end 101.6785 85.852) (width 0.25) (layer F.Cu) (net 4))
 (segment (start 103.632 82.169) (end 103.632 83.8985) (width 0.25) (layer F.Cu) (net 4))
 (segment (start 104.394 81.407) (end 103.632 82.169) (width 0.25) (layer F.Cu) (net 4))
 (segment (start 104.399001 81.412001) (end 104.394 81.407) (width 0.25) (layer F.Cu) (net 4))
 (segment (start 107.442 80.137) (end 106.166999 81.412001) (width 0.25) (layer F.Cu) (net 4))
 (segment (start 106.166999 81.412001) (end 104.399001 81.412001) (width 0.25) (layer F.Cu) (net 4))
 (segment (start 101.6785 86.7387) (end 98.7298 89.6874) (width 0.25) (layer F.Cu) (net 4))
 (segment (start 101.6785 85.807) (end 101.6785 86.7387) (width 0.25) (layer F.Cu) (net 4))
 (segment (start 106.5335 86.607) (end 108.839 88.9125) (width 0.25) (layer F.Cu) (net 6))
 (segment (start 106.5335 85.807) (end 106.5335 86.607) (width 0.25) (layer F.Cu) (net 6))
 (segment (start 108.839 88.9125) (end 108.839 90.297) (width 0.25) (layer F.Cu) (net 6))
 (segment (start 108.839 90.297) (end 109.855 91.313) (width 0.25) (layer F.Cu) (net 6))
 (segment (start 109.855 91.313) (end 113.284 91.313) (width 0.25) (layer F.Cu) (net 6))
 (segment (start 113.284 91.313) (end 114.808 92.837) (width 0.25) (layer F.Cu) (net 6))
 (segment (start 106.5335 85.007) (end 106.5335 85.807) (width 0.25) (layer F.Cu) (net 6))
 (segment (start 106.172 84.6455) (end 106.5335 85.007) (width 0.25) (layer F.Cu) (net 6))
 (segment (start 106.172 82.207998) (end 106.172 84.6455) (width 0.25) (layer F.Cu) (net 6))
 (segment (start 106.977999 81.401999) (end 106.172 82.207998) (width 0.25) (layer F.Cu) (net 6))
 (segment (start 111.246999 81.401999) (end 106.977999 81.401999) (width 0.25) (layer F.Cu) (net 6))
 (segment (start 112.522 82.677) (end 111.246999 81.401999) (width 0.25) (layer F.Cu) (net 6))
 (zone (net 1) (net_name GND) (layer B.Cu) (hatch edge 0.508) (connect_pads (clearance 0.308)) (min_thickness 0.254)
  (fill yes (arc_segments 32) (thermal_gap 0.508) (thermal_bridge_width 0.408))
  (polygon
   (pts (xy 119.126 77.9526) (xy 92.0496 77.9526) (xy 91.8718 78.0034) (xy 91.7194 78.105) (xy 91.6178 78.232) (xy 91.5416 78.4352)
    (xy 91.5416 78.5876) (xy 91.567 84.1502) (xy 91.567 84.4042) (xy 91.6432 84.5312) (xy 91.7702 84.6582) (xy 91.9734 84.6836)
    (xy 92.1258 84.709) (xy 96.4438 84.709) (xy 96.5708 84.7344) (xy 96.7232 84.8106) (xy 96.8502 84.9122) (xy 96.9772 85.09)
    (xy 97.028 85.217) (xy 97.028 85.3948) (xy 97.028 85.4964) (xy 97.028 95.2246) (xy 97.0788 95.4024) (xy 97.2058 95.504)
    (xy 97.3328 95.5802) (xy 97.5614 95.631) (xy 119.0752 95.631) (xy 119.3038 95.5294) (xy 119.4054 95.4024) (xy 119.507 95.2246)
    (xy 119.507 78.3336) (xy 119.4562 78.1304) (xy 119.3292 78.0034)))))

